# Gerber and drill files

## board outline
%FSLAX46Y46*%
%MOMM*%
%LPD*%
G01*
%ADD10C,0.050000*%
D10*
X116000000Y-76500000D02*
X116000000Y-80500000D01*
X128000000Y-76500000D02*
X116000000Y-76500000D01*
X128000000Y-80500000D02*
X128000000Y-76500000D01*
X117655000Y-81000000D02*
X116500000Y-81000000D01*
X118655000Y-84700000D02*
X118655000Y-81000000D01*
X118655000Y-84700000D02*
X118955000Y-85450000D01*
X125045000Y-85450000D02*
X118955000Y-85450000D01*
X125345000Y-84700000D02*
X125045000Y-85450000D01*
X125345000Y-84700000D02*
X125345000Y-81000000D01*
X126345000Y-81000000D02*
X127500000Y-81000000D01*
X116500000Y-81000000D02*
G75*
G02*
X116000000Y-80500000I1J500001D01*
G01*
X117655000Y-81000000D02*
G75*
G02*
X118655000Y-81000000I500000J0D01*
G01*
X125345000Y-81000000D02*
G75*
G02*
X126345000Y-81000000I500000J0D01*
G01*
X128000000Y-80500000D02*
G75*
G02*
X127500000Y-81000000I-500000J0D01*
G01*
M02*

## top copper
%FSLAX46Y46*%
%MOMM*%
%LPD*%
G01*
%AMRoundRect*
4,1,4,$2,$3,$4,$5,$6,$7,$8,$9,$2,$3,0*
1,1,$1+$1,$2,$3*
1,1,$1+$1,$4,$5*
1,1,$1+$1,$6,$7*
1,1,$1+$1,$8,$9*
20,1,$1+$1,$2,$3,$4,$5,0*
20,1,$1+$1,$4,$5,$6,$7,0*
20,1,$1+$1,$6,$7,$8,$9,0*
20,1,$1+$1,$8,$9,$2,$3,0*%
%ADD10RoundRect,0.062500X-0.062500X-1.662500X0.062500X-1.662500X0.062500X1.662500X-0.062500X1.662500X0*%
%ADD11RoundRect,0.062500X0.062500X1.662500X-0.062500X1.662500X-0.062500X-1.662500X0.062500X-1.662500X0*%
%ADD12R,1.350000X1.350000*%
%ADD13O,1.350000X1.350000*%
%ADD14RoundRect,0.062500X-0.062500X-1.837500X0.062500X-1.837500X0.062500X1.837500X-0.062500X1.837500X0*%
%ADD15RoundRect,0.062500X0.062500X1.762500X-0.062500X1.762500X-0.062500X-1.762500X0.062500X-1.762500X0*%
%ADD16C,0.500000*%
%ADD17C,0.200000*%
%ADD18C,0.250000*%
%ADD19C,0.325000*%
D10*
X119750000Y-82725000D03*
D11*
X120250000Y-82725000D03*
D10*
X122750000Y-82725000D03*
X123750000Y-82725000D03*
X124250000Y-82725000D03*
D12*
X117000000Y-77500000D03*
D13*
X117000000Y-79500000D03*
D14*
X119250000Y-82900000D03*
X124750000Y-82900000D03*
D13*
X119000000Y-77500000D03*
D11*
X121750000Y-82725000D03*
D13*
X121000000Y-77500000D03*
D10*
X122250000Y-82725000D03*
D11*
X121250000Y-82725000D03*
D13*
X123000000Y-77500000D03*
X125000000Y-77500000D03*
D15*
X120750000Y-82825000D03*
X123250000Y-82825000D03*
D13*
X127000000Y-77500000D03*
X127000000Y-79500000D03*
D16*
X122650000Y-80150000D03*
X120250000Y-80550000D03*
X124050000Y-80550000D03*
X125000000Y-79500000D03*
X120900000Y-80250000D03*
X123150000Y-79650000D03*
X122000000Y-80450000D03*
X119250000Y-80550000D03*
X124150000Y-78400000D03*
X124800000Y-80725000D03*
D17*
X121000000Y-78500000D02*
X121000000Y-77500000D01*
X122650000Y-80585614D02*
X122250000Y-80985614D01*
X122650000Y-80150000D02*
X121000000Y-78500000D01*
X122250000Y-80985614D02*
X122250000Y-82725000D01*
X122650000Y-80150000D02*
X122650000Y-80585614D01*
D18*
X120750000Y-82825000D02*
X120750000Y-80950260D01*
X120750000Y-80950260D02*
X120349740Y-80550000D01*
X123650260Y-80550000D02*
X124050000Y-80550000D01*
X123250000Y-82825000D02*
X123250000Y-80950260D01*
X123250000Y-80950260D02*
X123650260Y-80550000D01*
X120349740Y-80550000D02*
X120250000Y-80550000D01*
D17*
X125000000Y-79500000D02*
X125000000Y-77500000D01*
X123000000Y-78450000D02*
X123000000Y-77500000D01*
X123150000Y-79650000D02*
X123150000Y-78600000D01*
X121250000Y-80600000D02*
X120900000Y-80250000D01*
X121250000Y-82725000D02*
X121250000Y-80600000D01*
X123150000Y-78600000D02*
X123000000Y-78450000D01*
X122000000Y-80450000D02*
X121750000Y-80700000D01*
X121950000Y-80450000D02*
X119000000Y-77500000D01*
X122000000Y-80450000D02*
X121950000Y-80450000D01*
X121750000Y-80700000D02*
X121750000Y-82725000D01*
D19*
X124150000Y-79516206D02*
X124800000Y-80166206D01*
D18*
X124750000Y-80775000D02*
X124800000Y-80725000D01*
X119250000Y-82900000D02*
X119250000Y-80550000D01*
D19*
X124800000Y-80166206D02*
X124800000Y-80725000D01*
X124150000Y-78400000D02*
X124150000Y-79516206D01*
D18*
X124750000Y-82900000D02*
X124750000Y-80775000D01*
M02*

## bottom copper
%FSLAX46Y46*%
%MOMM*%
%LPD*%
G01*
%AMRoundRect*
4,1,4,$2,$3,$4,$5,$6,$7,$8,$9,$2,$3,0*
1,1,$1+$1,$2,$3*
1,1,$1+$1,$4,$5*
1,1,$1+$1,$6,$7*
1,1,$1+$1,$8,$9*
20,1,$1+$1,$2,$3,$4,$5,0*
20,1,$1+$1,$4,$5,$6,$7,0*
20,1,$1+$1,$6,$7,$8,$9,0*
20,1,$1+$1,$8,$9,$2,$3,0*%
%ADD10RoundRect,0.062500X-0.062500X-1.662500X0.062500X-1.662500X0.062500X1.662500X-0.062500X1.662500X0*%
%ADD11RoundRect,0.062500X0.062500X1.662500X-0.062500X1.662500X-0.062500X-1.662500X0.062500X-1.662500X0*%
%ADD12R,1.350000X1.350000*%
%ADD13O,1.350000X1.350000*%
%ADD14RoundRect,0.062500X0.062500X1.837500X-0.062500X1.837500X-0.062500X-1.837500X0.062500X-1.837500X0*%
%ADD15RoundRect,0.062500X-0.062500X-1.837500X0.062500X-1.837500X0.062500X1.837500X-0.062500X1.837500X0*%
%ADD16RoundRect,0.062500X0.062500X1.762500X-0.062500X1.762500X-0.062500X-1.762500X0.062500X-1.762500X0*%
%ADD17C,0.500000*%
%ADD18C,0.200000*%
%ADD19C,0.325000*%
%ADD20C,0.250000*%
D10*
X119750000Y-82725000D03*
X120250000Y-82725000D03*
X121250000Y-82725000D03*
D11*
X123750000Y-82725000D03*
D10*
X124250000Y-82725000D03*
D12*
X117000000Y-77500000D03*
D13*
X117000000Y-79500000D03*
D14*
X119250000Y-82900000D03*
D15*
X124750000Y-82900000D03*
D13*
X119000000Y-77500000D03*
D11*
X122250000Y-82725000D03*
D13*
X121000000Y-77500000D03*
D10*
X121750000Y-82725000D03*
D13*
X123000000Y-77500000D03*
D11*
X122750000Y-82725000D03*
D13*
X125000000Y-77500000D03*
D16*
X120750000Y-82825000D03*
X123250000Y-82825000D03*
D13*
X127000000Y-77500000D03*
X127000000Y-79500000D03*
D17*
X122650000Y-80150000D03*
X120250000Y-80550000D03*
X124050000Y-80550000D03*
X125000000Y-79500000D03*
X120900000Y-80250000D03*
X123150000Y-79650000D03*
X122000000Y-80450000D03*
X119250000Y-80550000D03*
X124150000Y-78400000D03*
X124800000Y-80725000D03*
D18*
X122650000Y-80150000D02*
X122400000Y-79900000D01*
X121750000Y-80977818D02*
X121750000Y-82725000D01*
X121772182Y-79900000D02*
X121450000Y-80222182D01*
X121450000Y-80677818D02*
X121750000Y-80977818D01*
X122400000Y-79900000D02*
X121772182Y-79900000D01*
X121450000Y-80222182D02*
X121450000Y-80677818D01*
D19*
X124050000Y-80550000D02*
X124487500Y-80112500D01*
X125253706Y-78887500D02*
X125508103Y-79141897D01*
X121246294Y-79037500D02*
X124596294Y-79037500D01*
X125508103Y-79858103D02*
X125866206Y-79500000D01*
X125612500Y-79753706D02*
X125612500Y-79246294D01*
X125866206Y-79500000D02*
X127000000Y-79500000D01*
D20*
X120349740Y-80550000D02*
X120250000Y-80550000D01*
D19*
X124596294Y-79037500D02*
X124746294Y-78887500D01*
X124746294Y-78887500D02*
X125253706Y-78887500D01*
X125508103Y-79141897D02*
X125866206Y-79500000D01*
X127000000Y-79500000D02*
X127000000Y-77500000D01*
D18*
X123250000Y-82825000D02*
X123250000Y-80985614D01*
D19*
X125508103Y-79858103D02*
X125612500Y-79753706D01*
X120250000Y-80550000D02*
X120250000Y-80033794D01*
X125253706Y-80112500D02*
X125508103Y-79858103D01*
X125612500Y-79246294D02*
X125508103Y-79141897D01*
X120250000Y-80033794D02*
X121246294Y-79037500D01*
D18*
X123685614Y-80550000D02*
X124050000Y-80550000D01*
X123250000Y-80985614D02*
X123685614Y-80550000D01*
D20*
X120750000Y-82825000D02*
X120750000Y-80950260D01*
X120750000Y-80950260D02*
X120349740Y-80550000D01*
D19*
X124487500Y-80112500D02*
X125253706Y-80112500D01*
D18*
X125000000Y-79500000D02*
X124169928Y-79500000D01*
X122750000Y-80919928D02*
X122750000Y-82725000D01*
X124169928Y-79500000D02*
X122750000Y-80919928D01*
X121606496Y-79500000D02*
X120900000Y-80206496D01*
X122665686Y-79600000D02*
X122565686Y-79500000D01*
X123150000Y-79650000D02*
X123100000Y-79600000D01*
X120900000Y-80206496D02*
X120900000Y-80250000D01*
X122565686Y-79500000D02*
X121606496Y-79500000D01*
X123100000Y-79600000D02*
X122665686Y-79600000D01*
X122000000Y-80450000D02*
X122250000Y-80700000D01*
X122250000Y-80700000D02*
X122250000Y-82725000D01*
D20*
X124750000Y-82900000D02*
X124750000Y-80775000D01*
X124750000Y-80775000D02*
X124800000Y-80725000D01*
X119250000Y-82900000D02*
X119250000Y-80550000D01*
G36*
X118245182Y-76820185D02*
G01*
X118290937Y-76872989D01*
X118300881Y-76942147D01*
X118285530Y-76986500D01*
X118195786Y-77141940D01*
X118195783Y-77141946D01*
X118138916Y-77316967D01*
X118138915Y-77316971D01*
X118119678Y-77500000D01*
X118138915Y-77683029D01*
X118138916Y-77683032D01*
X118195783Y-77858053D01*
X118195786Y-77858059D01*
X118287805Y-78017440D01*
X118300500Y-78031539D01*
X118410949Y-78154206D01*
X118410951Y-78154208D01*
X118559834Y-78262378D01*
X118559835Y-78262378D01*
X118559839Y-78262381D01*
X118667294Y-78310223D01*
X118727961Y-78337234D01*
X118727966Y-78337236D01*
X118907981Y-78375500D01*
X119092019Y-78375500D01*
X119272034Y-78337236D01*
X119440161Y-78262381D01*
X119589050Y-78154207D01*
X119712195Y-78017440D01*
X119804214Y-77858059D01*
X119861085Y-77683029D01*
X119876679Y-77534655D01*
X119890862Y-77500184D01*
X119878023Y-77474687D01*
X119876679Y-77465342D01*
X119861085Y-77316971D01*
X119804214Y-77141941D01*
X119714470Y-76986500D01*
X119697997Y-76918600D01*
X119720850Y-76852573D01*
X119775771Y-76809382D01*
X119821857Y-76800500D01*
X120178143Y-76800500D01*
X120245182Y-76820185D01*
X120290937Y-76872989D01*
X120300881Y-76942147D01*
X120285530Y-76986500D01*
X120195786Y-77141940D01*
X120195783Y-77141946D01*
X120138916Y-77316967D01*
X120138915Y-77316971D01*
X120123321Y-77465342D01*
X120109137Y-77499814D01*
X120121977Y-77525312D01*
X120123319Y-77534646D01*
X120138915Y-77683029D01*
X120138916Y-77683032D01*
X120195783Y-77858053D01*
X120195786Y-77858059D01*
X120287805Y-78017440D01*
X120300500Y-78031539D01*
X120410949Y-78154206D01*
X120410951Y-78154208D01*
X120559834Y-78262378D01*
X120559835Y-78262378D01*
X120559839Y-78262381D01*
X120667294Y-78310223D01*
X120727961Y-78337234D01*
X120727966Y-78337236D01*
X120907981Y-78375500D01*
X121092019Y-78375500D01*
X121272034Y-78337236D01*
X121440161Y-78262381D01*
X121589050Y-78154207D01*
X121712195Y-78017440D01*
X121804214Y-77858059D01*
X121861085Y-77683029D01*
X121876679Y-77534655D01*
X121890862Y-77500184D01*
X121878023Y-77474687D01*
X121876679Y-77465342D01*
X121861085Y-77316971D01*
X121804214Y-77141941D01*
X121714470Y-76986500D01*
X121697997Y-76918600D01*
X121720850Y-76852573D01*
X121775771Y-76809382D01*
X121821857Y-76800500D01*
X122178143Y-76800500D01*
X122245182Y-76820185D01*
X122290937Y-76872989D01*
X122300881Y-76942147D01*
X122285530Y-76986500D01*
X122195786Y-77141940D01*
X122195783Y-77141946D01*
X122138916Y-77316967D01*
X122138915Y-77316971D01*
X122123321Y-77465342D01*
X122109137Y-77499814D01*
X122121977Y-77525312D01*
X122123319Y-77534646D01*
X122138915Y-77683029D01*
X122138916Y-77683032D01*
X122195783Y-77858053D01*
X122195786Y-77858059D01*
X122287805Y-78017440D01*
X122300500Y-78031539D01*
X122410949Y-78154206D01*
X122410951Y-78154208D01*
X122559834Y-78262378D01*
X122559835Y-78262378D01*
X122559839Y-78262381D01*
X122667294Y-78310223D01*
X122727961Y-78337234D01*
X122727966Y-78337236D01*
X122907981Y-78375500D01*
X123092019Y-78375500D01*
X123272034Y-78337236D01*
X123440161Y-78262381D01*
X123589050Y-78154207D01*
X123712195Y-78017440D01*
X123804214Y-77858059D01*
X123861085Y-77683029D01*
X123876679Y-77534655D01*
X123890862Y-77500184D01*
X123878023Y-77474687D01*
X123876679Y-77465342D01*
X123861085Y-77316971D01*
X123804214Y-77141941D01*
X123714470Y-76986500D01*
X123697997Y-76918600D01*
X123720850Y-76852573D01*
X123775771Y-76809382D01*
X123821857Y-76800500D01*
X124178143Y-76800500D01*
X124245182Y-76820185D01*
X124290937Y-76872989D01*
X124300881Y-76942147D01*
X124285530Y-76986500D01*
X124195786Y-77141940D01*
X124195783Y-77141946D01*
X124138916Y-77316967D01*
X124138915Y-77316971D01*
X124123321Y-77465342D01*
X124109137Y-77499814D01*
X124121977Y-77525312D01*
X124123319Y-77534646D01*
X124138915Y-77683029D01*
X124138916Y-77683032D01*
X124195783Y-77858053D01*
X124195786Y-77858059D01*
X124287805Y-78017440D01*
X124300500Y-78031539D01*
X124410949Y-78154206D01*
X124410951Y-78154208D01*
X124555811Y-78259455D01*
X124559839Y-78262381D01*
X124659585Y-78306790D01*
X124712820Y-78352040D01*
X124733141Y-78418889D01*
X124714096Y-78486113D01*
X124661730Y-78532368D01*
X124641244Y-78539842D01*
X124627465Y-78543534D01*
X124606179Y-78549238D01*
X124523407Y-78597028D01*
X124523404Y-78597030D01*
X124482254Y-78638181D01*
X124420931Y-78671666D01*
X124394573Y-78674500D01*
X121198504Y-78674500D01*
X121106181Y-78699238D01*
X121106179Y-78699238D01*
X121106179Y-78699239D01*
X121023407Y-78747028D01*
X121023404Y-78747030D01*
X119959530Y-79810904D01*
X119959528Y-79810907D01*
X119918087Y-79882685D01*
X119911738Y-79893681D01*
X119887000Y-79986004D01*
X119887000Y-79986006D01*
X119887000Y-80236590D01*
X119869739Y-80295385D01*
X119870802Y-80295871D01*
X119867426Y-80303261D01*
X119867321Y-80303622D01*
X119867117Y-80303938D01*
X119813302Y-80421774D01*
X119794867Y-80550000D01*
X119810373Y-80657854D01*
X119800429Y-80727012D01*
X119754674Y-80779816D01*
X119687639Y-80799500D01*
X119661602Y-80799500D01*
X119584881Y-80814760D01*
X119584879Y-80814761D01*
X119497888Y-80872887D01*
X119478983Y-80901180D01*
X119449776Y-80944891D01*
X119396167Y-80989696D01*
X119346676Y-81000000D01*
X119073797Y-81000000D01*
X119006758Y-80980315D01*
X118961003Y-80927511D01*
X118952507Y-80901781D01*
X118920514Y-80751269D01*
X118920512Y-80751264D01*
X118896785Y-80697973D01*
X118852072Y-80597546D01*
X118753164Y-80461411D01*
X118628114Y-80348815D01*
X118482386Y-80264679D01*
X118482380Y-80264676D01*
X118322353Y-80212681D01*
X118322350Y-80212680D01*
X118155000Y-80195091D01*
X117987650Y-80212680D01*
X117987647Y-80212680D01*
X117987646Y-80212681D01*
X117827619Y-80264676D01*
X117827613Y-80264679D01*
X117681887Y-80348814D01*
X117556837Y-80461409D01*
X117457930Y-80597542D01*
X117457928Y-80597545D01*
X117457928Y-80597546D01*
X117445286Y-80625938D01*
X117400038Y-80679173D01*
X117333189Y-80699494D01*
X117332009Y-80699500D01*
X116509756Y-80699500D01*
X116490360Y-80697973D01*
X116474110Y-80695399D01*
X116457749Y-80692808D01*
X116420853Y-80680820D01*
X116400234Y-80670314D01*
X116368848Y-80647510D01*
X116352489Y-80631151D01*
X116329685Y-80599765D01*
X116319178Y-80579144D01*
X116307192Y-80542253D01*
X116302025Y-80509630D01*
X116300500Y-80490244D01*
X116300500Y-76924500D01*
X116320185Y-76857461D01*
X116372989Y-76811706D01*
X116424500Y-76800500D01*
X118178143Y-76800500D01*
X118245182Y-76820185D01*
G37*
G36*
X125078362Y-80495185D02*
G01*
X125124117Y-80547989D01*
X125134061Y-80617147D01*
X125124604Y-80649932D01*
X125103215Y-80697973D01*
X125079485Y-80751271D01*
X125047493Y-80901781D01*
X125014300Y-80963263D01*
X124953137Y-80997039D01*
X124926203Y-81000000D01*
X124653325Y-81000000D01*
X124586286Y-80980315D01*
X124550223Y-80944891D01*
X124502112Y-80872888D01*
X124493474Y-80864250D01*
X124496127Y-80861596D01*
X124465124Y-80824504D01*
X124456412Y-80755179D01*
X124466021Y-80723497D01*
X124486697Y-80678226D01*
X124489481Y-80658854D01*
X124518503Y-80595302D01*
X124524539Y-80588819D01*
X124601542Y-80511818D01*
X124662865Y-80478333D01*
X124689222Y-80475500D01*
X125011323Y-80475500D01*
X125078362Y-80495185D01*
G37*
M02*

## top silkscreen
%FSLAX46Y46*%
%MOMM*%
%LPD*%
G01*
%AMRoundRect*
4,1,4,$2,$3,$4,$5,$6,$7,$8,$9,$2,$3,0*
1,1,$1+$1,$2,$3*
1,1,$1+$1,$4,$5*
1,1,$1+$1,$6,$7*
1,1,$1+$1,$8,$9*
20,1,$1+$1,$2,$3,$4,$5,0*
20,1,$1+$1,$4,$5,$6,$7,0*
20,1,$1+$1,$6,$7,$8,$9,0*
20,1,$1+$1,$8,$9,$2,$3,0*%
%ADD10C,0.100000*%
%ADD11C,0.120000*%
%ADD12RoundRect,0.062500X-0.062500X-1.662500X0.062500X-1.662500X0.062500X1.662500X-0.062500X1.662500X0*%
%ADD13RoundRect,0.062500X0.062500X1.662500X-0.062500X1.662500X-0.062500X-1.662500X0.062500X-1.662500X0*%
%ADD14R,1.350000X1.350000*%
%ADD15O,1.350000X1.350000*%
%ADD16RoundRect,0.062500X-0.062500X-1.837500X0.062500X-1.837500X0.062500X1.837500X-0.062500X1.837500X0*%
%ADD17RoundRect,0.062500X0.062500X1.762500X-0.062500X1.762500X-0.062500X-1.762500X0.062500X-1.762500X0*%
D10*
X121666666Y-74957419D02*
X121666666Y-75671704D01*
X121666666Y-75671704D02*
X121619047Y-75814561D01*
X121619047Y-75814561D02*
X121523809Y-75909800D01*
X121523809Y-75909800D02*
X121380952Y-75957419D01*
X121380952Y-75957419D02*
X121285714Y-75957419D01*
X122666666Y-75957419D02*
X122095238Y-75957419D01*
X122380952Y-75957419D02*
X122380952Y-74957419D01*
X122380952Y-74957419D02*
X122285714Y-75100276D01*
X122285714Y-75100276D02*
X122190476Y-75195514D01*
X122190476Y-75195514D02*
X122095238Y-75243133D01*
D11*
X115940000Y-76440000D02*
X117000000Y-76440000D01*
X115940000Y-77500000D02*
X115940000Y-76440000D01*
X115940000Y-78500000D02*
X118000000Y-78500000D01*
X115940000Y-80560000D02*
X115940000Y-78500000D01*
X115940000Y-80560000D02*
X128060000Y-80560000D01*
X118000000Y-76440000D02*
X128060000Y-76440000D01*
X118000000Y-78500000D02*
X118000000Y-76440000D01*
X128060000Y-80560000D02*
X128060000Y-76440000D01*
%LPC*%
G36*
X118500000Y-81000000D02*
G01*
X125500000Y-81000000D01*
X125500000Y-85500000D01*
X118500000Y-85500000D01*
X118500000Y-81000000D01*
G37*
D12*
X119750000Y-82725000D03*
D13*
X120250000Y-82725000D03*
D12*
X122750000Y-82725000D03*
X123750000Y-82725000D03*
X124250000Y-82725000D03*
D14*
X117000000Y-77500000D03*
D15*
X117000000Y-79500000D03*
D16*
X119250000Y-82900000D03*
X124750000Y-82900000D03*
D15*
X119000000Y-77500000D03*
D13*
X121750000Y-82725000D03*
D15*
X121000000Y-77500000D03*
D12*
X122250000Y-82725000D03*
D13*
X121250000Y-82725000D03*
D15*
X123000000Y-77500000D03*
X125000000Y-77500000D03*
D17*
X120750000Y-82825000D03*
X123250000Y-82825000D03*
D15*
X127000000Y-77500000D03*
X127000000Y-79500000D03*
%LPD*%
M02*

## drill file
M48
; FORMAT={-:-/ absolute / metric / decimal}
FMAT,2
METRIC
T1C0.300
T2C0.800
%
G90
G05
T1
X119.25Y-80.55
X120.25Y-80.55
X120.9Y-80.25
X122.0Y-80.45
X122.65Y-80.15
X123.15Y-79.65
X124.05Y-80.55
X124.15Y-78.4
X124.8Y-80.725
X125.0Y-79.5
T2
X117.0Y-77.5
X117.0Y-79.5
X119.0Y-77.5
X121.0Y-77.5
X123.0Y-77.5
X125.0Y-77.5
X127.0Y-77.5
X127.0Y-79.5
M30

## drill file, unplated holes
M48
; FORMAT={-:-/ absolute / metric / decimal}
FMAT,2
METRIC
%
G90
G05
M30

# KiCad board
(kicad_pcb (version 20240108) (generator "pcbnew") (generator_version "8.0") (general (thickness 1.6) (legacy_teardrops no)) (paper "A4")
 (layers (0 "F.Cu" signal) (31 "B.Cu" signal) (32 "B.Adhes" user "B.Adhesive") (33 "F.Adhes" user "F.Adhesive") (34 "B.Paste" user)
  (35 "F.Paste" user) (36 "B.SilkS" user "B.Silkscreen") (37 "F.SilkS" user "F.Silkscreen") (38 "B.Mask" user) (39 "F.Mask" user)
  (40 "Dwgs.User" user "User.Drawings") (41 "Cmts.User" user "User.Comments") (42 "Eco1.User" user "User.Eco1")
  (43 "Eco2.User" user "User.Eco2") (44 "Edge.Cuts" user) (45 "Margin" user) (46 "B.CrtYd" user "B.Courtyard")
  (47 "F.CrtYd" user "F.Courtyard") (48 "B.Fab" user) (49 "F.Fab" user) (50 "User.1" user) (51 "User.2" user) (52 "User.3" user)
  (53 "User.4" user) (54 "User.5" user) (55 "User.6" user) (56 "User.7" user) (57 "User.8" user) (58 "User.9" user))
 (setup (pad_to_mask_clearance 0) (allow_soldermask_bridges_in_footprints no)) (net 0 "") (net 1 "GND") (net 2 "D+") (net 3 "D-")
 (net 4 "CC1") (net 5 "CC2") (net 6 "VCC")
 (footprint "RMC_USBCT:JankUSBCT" (layer "F.Cu") (at 122 81)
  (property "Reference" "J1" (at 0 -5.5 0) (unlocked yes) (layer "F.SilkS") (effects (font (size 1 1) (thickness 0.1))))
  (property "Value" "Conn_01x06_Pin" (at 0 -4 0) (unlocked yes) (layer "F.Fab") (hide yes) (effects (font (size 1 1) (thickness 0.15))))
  (fp_line (start -6.06 -4.56) (end -5 -4.56) (stroke (width 0.12) (type solid)) (layer "F.SilkS"))
  (fp_line (start -6.06 -3.5) (end -6.06 -4.56) (stroke (width 0.12) (type solid)) (layer "F.SilkS"))
  (fp_line (start -6.06 -2.5) (end -4 -2.5) (stroke (width 0.12) (type solid)) (layer "F.SilkS"))
  (fp_line (start -6.06 -0.44) (end -6.06 -2.5) (stroke (width 0.12) (type solid)) (layer "F.SilkS"))
  (fp_line (start -6.06 -0.44) (end 6.06 -0.44) (stroke (width 0.12) (type solid)) (layer "F.SilkS"))
  (fp_line (start -4 -4.56) (end 6.06 -4.56) (stroke (width 0.12) (type solid)) (layer "F.SilkS"))
  (fp_line (start -4 -2.5) (end -4 -4.56) (stroke (width 0.12) (type solid)) (layer "F.SilkS"))
  (fp_line (start 6.06 -0.44) (end 6.06 -4.56) (stroke (width 0.12) (type solid)) (layer "F.SilkS"))
  (fp_line (start -4.345 0) (end -5.5 0) (stroke (width 0.05) (type default)) (layer "Edge.Cuts"))
  (fp_line (start -3.345 3.7) (end -3.345 0) (stroke (width 0.05) (type default)) (layer "Edge.Cuts"))
  (fp_line (start -3.345 3.7) (end -3.045 4.45) (stroke (width 0.05) (type default)) (layer "Edge.Cuts"))
  (fp_line (start 3.045 4.45) (end -3.045 4.45) (stroke (width 0.05) (type default)) (layer "Edge.Cuts"))
  (fp_line (start 3.345 3.7) (end 3.045 4.45) (stroke (width 0.05) (type default)) (layer "Edge.Cuts"))
  (fp_line (start 3.345 3.7) (end 3.345 0) (stroke (width 0.05) (type default)) (layer "Edge.Cuts"))
  (fp_line (start 4.345 0) (end 5.5 0) (stroke (width 0.05) (type default)) (layer "Edge.Cuts"))
  (fp_arc (start -5.5 0) (mid -5.853553 -0.146447) (end -6 -0.5) (stroke (width 0.05) (type default)) (layer "Edge.Cuts"))
  (fp_arc (start -4.345 0) (mid -3.845 -0.5) (end -3.345 0) (stroke (width 0.05) (type default)) (layer "Edge.Cuts"))
  (fp_arc (start 3.345 0) (mid 3.845 -0.5) (end 4.345 0) (stroke (width 0.05) (type default)) (layer "Edge.Cuts"))
  (fp_arc (start 6 -0.5) (mid 5.853553 -0.146447) (end 5.5 0) (stroke (width 0.05) (type default)) (layer "Edge.Cuts"))
  (pad "" smd roundrect (at -2.25 1.725) (size 0.25 3.45) (layers "F.Cu" "F.Paste" "F.Mask") (roundrect_rratio 0.25)
   (thermal_bridge_angle 45))
  (pad "" smd roundrect (at -2.25 1.725) (size 0.25 3.45) (layers "B.Cu" "B.Paste" "B.Mask") (roundrect_rratio 0.25)
   (thermal_bridge_angle 45))
  (pad "" smd roundrect (at -1.75 1.725 180) (size 0.25 3.45) (layers "F.Cu" "F.Paste" "F.Mask") (roundrect_rratio 0.25)
   (thermal_bridge_angle 45))
  (pad "" smd roundrect (at -1.75 1.725) (size 0.25 3.45) (layers "B.Cu" "B.Paste" "B.Mask") (roundrect_rratio 0.25)
   (thermal_bridge_angle 45))
  (pad "" smd roundrect (at -0.75 1.725) (size 0.25 3.45) (layers "B.Cu" "B.Paste" "B.Mask") (roundrect_rratio 0.25)
   (thermal_bridge_angle 45))
  (pad "" smd roundrect (at 0.75 1.725) (size 0.25 3.45) (layers "F.Cu" "F.Paste" "F.Mask") (roundrect_rratio 0.25)
   (thermal_bridge_angle 45))
  (pad "" smd roundrect (at 1.75 1.725) (size 0.25 3.45) (layers "F.Cu" "F.Paste" "F.Mask") (roundrect_rratio 0.25)
   (thermal_bridge_angle 45))
  (pad "" smd roundrect (at 1.75 1.725 180) (size 0.25 3.45) (layers "B.Cu" "B.Paste" "B.Mask") (roundrect_rratio 0.25)
   (thermal_bridge_angle 45))
  (pad "" smd roundrect (at 2.25 1.725) (size 0.25 3.45) (layers "F.Cu" "F.Paste" "F.Mask") (roundrect_rratio 0.25)
   (thermal_bridge_angle 45))
  (pad "" smd roundrect (at 2.25 1.725) (size 0.25 3.45) (layers "B.Cu" "B.Paste" "B.Mask") (roundrect_rratio 0.25)
   (thermal_bridge_angle 45))
  (pad "1" thru_hole rect (at -5 -3.5 90) (size 1.35 1.35) (drill 0.8) (layers "*.Cu" "*.Mask") (remove_unused_layers no) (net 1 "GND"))
  (pad "1" thru_hole oval (at -5 -1.5 90) (size 1.35 1.35) (drill 0.8) (layers "*.Cu" "*.Mask") (remove_unused_layers no) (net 1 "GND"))
  (pad "1" smd roundrect (at -2.75 1.9) (size 0.25 3.8) (layers "F.Cu" "F.Paste" "F.Mask") (roundrect_rratio 0.25) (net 1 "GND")
   (thermal_bridge_angle 45))
  (pad "1" smd roundrect (at -2.75 1.9 180) (size 0.25 3.8) (layers "B.Cu" "B.Paste" "B.Mask") (roundrect_rratio 0.25) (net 1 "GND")
   (thermal_bridge_angle 45))
  (pad "1" smd roundrect (at 2.75 1.9) (size 0.25 3.8) (layers "F.Cu" "F.Paste" "F.Mask") (roundrect_rratio 0.25) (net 1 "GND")
   (thermal_bridge_angle 45))
  (pad "1" smd roundrect (at 2.75 1.9) (size 0.25 3.8) (layers "B.Cu" "B.Paste" "B.Mask") (roundrect_rratio 0.25) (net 1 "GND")
   (thermal_bridge_angle 45))
  (pad "2" thru_hole oval (at -3 -3.5 90) (size 1.35 1.35) (drill 0.8) (layers "*.Cu" "*.Mask") (remove_unused_layers no) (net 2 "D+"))
  (pad "2" smd roundrect (at -0.25 1.725 180) (size 0.25 3.45) (layers "F.Cu" "F.Paste" "F.Mask") (roundrect_rratio 0.25) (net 2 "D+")
   (thermal_bridge_angle 45))
  (pad "2" smd roundrect (at 0.25 1.725 180) (size 0.25 3.45) (layers "B.Cu" "B.Paste" "B.Mask") (roundrect_rratio 0.25) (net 2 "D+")
   (thermal_bridge_angle 45))
  (pad "3" thru_hole oval (at -1 -3.5 90) (size 1.35 1.35) (drill 0.8) (layers "*.Cu" "*.Mask") (remove_unused_layers no) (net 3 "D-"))
  (pad "3" smd roundrect (at -0.25 1.725) (size 0.25 3.45) (layers "B.Cu" "B.Paste" "B.Mask") (roundrect_rratio 0.25) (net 3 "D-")
   (thermal_bridge_angle 45))
  (pad "3" smd roundrect (at 0.25 1.725) (size 0.25 3.45) (layers "F.Cu" "F.Paste" "F.Mask") (roundrect_rratio 0.25) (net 3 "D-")
   (thermal_bridge_angle 45))
  (pad "4" smd roundrect (at -0.75 1.725 180) (size 0.25 3.45) (layers "F.Cu" "F.Paste" "F.Mask") (roundrect_rratio 0.25) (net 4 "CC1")
   (thermal_bridge_angle 45))
  (pad "4" thru_hole oval (at 1 -3.5 90) (size 1.35 1.35) (drill 0.8) (layers "*.Cu" "*.Mask") (remove_unused_layers no) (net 4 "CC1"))
  (pad "5" smd roundrect (at 0.75 1.725 180) (size 0.25 3.45) (layers "B.Cu" "B.Paste" "B.Mask") (roundrect_rratio 0.25) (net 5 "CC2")
   (thermal_bridge_angle 45))
  (pad "5" thru_hole oval (at 3 -3.5 90) (size 1.35 1.35) (drill 0.8) (layers "*.Cu" "*.Mask") (remove_unused_layers no) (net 5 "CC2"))
  (pad "6" smd roundrect (at -1.25 1.825 180) (size 0.25 3.65) (layers "F.Cu" "F.Paste" "F.Mask") (roundrect_rratio 0.25) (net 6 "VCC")
   (thermal_bridge_angle 45))
  (pad "6" smd roundrect (at -1.25 1.825 180) (size 0.25 3.65) (layers "B.Cu" "B.Paste" "B.Mask") (roundrect_rratio 0.25) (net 6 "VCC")
   (thermal_bridge_angle 45))
  (pad "6" smd roundrect (at 1.25 1.825 180) (size 0.25 3.65) (layers "F.Cu" "F.Paste" "F.Mask") (roundrect_rratio 0.25) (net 6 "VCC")
   (thermal_bridge_angle 45))
  (pad "6" smd roundrect (at 1.25 1.825 180) (size 0.25 3.65) (layers "B.Cu" "B.Paste" "B.Mask") (roundrect_rratio 0.25) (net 6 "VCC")
   (thermal_bridge_angle 45))
  (pad "6" thru_hole oval (at 5 -3.5 90) (size 1.35 1.35) (drill 0.8) (layers "*.Cu" "*.Mask") (remove_unused_layers no) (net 6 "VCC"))
  (pad "6" thru_hole oval (at 5 -1.5 90) (size 1.35 1.35) (drill 0.8) (layers "*.Cu" "*.Mask") (remove_unused_layers no) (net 6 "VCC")))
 (gr_line (start 116 76.5) (end 116 80.5) (stroke (width 0.05) (type default)) (layer "Edge.Cuts"))
 (gr_line (start 128 76.5) (end 116 76.5) (stroke (width 0.05) (type default)) (layer "Edge.Cuts"))
 (gr_line (start 128 80.5) (end 128 76.5) (stroke (width 0.05) (type default)) (layer "Edge.Cuts"))
 (segment (start 121 78.5) (end 121 77.5) (width 0.2) (layer "F.Cu") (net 3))
 (segment (start 122.65 80.585614) (end 122.25 80.985614) (width 0.2) (layer "F.Cu") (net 3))
 (segment (start 122.65 80.15) (end 121 78.5) (width 0.2) (layer "F.Cu") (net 3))
 (segment (start 122.25 80.985614) (end 122.25 82.725) (width 0.2) (layer "F.Cu") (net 3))
 (segment (start 122.65 80.15) (end 122.65 80.585614) (width 0.2) (layer "F.Cu") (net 3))
 (via (at 122.65 80.15) (size 0.5) (drill 0.3) (layers "F.Cu" "B.Cu") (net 3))
 (segment (start 122.65 80.15) (end 122.4 79.9) (width 0.2) (layer "B.Cu") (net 3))
 (segment (start 121.75 80.977818) (end 121.75 82.725) (width 0.2) (layer "B.Cu") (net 3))
 (segment (start 121.772182 79.9) (end 121.45 80.222182) (width 0.2) (layer "B.Cu") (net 3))
 (segment (start 121.45 80.677818) (end 121.75 80.977818) (width 0.2) (layer "B.Cu") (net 3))
 (segment (start 122.4 79.9) (end 121.772182 79.9) (width 0.2) (layer "B.Cu") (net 3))
 (segment (start 121.45 80.222182) (end 121.45 80.677818) (width 0.2) (layer "B.Cu") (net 3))
 (segment (start 120.75 82.825) (end 120.75 80.95026) (width 0.25) (layer "F.Cu") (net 6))
 (segment (start 120.75 80.95026) (end 120.34974 80.55) (width 0.25) (layer "F.Cu") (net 6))
 (segment (start 123.65026 80.55) (end 124.05 80.55) (width 0.25) (layer "F.Cu") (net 6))
 (segment (start 123.25 82.825) (end 123.25 80.95026) (width 0.25) (layer "F.Cu") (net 6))
 (segment (start 123.25 80.95026) (end 123.65026 80.55) (width 0.25) (layer "F.Cu") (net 6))
 (segment (start 120.34974 80.55) (end 120.25 80.55) (width 0.25) (layer "F.Cu") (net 6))
 (via (at 120.25 80.55) (size 0.5) (drill 0.3) (layers "F.Cu" "B.Cu") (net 6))
 (via (at 124.05 80.55) (size 0.5) (drill 0.3) (layers "F.Cu" "B.Cu") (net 6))
 (segment (start 124.05 80.55) (end 124.4875 80.1125) (width 0.325) (layer "B.Cu") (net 6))
 (segment (start 125.253706 78.8875) (end 125.508103 79.141897) (width 0.325) (layer "B.Cu") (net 6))
 (segment (start 121.246294 79.0375) (end 124.596294 79.0375) (width 0.325) (layer "B.Cu") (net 6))
 (segment (start 125.508103 79.858103) (end 125.866206 79.5) (width 0.325) (layer "B.Cu") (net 6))
 (segment (start 125.6125 79.753706) (end 125.6125 79.246294) (width 0.325) (layer "B.Cu") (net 6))
 (segment (start 125.866206 79.5) (end 127 79.5) (width 0.325) (layer "B.Cu") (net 6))
 (segment (start 120.34974 80.55) (end 120.25 80.55) (width 0.25) (layer "B.Cu") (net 6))
 (segment (start 124.596294 79.0375) (end 124.746294 78.8875) (width 0.325) (layer "B.Cu") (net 6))
 (segment (start 124.746294 78.8875) (end 125.253706 78.8875) (width 0.325) (layer "B.Cu") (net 6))
 (segment (start 125.508103 79.141897) (end 125.866206 79.5) (width 0.325) (layer "B.Cu") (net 6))
 (segment (start 127 79.5) (end 127 77.5) (width 0.325) (layer "B.Cu") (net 6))
 (segment (start 123.25 82.825) (end 123.25 80.985614) (width 0.2) (layer "B.Cu") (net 6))
 (segment (start 125.508103 79.858103) (end 125.6125 79.753706) (width 0.325) (layer "B.Cu") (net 6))
 (segment (start 120.25 80.55) (end 120.25 80.033794) (width 0.325) (layer "B.Cu") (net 6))
 (segment (start 125.253706 80.1125) (end 125.508103 79.858103) (width 0.325) (layer "B.Cu") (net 6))
 (segment (start 125.6125 79.246294) (end 125.508103 79.141897) (width 0.325) (layer "B.Cu") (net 6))
 (segment (start 120.25 80.033794) (end 121.246294 79.0375) (width 0.325) (layer "B.Cu") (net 6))
 (segment (start 123.685614 80.55) (end 124.05 80.55) (width 0.2) (layer "B.Cu") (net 6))
 (segment (start 123.25 80.985614) (end 123.685614 80.55) (width 0.2) (layer "B.Cu") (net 6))
 (segment (start 120.75 82.825) (end 120.75 80.95026) (width 0.25) (layer "B.Cu") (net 6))
 (segment (start 120.75 80.95026) (end 120.34974 80.55) (width 0.25) (layer "B.Cu") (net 6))
 (segment (start 124.4875 80.1125) (end 125.253706 80.1125) (width 0.325) (layer "B.Cu") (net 6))
 (segment (start 125 79.5) (end 125 77.5) (width 0.2) (layer "F.Cu") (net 5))
 (via (at 125 79.5) (size 0.5) (drill 0.3) (layers "F.Cu" "B.Cu") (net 5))
 (segment (start 125 79.5) (end 124.169928 79.5) (width 0.2) (layer "B.Cu") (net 5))
 (segment (start 122.75 80.919928) (end 122.75 82.725) (width 0.2) (layer "B.Cu") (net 5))
 (segment (start 124.169928 79.5) (end 122.75 80.919928) (width 0.2) (layer "B.Cu") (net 5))
 (segment (start 123 78.45) (end 123 77.5) (width 0.2) (layer "F.Cu") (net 4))
 (segment (start 123.15 79.65) (end 123.15 78.6) (width 0.2) (layer "F.Cu") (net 4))
 (segment (start 121.25 80.6) (end 120.9 80.25) (width 0.2) (layer "F.Cu") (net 4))
 (segment (start 121.25 82.725) (end 121.25 80.6) (width 0.2) (layer "F.Cu") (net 4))
 (segment (start 123.15 78.6) (end 123 78.45) (width 0.2) (layer "F.Cu") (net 4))
 (via (at 120.9 80.25) (size 0.5) (drill 0.3) (layers "F.Cu" "B.Cu") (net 4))
 (via (at 123.15 79.65) (size 0.5) (drill 0.3) (layers "F.Cu" "B.Cu") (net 4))
 (segment (start 121.606496 79.5) (end 120.9 80.206496) (width 0.2) (layer "B.Cu") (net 4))
 (segment (start 122.665686 79.6) (end 122.565686 79.5) (width 0.2) (layer "B.Cu") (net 4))
 (segment (start 123.15 79.65) (end 123.1 79.6) (width 0.2) (layer "B.Cu") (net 4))
 (segment (start 120.9 80.206496) (end 120.9 80.25) (width 0.2) (layer "B.Cu") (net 4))
 (segment (start 122.565686 79.5) (end 121.606496 79.5) (width 0.2) (layer "B.Cu") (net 4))
 (segment (start 123.1 79.6) (end 122.665686 79.6) (width 0.2) (layer "B.Cu") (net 4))
 (segment (start 122 80.45) (end 121.75 80.7) (width 0.2) (layer "F.Cu") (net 2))
 (segment (start 121.95 80.45) (end 119 77.5) (width 0.2) (layer "F.Cu") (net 2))
 (segment (start 122 80.45) (end 121.95 80.45) (width 0.2) (layer "F.Cu") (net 2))
 (segment (start 121.75 80.7) (end 121.75 82.725) (width 0.2) (layer "F.Cu") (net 2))
 (via (at 122 80.45) (size 0.5) (drill 0.3) (layers "F.Cu" "B.Cu") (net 2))
 (segment (start 122 80.45) (end 122.25 80.7) (width 0.2) (layer "B.Cu") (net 2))
 (segment (start 122.25 80.7) (end 122.25 82.725) (width 0.2) (layer "B.Cu") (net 2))
 (segment (start 124.15 79.516206) (end 124.8 80.166206) (width 0.325) (layer "F.Cu") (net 1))
 (segment (start 124.75 80.775) (end 124.8 80.725) (width 0.25) (layer "F.Cu") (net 1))
 (segment (start 119.25 82.9) (end 119.25 80.55) (width 0.25) (layer "F.Cu") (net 1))
 (segment (start 124.8 80.166206) (end 124.8 80.725) (width 0.325) (layer "F.Cu") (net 1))
 (segment (start 124.15 78.4) (end 124.15 79.516206) (width 0.325) (layer "F.Cu") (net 1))
 (segment (start 124.75 82.9) (end 124.75 80.775) (width 0.25) (layer "F.Cu") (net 1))
 (via (at 119.25 80.55) (size 0.5) (drill 0.3) (layers "F.Cu" "B.Cu") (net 1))
 (via (at 124.15 78.4) (size 0.5) (drill 0.3) (layers "F.Cu" "B.Cu") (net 1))
 (via (at 124.8 80.725) (size 0.5) (drill 0.3) (layers "F.Cu" "B.Cu") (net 1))
 (segment (start 124.75 82.9) (end 124.75 80.775) (width 0.25) (layer "B.Cu") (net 1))
 (segment (start 124.75 80.775) (end 124.8 80.725) (width 0.25) (layer "B.Cu") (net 1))
 (segment (start 119.25 82.9) (end 119.25 80.55) (width 0.25) (layer "B.Cu") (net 1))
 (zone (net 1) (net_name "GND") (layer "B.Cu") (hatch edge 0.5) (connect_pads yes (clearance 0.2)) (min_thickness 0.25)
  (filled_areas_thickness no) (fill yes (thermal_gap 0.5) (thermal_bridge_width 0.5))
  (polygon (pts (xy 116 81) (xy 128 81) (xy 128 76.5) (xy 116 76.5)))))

